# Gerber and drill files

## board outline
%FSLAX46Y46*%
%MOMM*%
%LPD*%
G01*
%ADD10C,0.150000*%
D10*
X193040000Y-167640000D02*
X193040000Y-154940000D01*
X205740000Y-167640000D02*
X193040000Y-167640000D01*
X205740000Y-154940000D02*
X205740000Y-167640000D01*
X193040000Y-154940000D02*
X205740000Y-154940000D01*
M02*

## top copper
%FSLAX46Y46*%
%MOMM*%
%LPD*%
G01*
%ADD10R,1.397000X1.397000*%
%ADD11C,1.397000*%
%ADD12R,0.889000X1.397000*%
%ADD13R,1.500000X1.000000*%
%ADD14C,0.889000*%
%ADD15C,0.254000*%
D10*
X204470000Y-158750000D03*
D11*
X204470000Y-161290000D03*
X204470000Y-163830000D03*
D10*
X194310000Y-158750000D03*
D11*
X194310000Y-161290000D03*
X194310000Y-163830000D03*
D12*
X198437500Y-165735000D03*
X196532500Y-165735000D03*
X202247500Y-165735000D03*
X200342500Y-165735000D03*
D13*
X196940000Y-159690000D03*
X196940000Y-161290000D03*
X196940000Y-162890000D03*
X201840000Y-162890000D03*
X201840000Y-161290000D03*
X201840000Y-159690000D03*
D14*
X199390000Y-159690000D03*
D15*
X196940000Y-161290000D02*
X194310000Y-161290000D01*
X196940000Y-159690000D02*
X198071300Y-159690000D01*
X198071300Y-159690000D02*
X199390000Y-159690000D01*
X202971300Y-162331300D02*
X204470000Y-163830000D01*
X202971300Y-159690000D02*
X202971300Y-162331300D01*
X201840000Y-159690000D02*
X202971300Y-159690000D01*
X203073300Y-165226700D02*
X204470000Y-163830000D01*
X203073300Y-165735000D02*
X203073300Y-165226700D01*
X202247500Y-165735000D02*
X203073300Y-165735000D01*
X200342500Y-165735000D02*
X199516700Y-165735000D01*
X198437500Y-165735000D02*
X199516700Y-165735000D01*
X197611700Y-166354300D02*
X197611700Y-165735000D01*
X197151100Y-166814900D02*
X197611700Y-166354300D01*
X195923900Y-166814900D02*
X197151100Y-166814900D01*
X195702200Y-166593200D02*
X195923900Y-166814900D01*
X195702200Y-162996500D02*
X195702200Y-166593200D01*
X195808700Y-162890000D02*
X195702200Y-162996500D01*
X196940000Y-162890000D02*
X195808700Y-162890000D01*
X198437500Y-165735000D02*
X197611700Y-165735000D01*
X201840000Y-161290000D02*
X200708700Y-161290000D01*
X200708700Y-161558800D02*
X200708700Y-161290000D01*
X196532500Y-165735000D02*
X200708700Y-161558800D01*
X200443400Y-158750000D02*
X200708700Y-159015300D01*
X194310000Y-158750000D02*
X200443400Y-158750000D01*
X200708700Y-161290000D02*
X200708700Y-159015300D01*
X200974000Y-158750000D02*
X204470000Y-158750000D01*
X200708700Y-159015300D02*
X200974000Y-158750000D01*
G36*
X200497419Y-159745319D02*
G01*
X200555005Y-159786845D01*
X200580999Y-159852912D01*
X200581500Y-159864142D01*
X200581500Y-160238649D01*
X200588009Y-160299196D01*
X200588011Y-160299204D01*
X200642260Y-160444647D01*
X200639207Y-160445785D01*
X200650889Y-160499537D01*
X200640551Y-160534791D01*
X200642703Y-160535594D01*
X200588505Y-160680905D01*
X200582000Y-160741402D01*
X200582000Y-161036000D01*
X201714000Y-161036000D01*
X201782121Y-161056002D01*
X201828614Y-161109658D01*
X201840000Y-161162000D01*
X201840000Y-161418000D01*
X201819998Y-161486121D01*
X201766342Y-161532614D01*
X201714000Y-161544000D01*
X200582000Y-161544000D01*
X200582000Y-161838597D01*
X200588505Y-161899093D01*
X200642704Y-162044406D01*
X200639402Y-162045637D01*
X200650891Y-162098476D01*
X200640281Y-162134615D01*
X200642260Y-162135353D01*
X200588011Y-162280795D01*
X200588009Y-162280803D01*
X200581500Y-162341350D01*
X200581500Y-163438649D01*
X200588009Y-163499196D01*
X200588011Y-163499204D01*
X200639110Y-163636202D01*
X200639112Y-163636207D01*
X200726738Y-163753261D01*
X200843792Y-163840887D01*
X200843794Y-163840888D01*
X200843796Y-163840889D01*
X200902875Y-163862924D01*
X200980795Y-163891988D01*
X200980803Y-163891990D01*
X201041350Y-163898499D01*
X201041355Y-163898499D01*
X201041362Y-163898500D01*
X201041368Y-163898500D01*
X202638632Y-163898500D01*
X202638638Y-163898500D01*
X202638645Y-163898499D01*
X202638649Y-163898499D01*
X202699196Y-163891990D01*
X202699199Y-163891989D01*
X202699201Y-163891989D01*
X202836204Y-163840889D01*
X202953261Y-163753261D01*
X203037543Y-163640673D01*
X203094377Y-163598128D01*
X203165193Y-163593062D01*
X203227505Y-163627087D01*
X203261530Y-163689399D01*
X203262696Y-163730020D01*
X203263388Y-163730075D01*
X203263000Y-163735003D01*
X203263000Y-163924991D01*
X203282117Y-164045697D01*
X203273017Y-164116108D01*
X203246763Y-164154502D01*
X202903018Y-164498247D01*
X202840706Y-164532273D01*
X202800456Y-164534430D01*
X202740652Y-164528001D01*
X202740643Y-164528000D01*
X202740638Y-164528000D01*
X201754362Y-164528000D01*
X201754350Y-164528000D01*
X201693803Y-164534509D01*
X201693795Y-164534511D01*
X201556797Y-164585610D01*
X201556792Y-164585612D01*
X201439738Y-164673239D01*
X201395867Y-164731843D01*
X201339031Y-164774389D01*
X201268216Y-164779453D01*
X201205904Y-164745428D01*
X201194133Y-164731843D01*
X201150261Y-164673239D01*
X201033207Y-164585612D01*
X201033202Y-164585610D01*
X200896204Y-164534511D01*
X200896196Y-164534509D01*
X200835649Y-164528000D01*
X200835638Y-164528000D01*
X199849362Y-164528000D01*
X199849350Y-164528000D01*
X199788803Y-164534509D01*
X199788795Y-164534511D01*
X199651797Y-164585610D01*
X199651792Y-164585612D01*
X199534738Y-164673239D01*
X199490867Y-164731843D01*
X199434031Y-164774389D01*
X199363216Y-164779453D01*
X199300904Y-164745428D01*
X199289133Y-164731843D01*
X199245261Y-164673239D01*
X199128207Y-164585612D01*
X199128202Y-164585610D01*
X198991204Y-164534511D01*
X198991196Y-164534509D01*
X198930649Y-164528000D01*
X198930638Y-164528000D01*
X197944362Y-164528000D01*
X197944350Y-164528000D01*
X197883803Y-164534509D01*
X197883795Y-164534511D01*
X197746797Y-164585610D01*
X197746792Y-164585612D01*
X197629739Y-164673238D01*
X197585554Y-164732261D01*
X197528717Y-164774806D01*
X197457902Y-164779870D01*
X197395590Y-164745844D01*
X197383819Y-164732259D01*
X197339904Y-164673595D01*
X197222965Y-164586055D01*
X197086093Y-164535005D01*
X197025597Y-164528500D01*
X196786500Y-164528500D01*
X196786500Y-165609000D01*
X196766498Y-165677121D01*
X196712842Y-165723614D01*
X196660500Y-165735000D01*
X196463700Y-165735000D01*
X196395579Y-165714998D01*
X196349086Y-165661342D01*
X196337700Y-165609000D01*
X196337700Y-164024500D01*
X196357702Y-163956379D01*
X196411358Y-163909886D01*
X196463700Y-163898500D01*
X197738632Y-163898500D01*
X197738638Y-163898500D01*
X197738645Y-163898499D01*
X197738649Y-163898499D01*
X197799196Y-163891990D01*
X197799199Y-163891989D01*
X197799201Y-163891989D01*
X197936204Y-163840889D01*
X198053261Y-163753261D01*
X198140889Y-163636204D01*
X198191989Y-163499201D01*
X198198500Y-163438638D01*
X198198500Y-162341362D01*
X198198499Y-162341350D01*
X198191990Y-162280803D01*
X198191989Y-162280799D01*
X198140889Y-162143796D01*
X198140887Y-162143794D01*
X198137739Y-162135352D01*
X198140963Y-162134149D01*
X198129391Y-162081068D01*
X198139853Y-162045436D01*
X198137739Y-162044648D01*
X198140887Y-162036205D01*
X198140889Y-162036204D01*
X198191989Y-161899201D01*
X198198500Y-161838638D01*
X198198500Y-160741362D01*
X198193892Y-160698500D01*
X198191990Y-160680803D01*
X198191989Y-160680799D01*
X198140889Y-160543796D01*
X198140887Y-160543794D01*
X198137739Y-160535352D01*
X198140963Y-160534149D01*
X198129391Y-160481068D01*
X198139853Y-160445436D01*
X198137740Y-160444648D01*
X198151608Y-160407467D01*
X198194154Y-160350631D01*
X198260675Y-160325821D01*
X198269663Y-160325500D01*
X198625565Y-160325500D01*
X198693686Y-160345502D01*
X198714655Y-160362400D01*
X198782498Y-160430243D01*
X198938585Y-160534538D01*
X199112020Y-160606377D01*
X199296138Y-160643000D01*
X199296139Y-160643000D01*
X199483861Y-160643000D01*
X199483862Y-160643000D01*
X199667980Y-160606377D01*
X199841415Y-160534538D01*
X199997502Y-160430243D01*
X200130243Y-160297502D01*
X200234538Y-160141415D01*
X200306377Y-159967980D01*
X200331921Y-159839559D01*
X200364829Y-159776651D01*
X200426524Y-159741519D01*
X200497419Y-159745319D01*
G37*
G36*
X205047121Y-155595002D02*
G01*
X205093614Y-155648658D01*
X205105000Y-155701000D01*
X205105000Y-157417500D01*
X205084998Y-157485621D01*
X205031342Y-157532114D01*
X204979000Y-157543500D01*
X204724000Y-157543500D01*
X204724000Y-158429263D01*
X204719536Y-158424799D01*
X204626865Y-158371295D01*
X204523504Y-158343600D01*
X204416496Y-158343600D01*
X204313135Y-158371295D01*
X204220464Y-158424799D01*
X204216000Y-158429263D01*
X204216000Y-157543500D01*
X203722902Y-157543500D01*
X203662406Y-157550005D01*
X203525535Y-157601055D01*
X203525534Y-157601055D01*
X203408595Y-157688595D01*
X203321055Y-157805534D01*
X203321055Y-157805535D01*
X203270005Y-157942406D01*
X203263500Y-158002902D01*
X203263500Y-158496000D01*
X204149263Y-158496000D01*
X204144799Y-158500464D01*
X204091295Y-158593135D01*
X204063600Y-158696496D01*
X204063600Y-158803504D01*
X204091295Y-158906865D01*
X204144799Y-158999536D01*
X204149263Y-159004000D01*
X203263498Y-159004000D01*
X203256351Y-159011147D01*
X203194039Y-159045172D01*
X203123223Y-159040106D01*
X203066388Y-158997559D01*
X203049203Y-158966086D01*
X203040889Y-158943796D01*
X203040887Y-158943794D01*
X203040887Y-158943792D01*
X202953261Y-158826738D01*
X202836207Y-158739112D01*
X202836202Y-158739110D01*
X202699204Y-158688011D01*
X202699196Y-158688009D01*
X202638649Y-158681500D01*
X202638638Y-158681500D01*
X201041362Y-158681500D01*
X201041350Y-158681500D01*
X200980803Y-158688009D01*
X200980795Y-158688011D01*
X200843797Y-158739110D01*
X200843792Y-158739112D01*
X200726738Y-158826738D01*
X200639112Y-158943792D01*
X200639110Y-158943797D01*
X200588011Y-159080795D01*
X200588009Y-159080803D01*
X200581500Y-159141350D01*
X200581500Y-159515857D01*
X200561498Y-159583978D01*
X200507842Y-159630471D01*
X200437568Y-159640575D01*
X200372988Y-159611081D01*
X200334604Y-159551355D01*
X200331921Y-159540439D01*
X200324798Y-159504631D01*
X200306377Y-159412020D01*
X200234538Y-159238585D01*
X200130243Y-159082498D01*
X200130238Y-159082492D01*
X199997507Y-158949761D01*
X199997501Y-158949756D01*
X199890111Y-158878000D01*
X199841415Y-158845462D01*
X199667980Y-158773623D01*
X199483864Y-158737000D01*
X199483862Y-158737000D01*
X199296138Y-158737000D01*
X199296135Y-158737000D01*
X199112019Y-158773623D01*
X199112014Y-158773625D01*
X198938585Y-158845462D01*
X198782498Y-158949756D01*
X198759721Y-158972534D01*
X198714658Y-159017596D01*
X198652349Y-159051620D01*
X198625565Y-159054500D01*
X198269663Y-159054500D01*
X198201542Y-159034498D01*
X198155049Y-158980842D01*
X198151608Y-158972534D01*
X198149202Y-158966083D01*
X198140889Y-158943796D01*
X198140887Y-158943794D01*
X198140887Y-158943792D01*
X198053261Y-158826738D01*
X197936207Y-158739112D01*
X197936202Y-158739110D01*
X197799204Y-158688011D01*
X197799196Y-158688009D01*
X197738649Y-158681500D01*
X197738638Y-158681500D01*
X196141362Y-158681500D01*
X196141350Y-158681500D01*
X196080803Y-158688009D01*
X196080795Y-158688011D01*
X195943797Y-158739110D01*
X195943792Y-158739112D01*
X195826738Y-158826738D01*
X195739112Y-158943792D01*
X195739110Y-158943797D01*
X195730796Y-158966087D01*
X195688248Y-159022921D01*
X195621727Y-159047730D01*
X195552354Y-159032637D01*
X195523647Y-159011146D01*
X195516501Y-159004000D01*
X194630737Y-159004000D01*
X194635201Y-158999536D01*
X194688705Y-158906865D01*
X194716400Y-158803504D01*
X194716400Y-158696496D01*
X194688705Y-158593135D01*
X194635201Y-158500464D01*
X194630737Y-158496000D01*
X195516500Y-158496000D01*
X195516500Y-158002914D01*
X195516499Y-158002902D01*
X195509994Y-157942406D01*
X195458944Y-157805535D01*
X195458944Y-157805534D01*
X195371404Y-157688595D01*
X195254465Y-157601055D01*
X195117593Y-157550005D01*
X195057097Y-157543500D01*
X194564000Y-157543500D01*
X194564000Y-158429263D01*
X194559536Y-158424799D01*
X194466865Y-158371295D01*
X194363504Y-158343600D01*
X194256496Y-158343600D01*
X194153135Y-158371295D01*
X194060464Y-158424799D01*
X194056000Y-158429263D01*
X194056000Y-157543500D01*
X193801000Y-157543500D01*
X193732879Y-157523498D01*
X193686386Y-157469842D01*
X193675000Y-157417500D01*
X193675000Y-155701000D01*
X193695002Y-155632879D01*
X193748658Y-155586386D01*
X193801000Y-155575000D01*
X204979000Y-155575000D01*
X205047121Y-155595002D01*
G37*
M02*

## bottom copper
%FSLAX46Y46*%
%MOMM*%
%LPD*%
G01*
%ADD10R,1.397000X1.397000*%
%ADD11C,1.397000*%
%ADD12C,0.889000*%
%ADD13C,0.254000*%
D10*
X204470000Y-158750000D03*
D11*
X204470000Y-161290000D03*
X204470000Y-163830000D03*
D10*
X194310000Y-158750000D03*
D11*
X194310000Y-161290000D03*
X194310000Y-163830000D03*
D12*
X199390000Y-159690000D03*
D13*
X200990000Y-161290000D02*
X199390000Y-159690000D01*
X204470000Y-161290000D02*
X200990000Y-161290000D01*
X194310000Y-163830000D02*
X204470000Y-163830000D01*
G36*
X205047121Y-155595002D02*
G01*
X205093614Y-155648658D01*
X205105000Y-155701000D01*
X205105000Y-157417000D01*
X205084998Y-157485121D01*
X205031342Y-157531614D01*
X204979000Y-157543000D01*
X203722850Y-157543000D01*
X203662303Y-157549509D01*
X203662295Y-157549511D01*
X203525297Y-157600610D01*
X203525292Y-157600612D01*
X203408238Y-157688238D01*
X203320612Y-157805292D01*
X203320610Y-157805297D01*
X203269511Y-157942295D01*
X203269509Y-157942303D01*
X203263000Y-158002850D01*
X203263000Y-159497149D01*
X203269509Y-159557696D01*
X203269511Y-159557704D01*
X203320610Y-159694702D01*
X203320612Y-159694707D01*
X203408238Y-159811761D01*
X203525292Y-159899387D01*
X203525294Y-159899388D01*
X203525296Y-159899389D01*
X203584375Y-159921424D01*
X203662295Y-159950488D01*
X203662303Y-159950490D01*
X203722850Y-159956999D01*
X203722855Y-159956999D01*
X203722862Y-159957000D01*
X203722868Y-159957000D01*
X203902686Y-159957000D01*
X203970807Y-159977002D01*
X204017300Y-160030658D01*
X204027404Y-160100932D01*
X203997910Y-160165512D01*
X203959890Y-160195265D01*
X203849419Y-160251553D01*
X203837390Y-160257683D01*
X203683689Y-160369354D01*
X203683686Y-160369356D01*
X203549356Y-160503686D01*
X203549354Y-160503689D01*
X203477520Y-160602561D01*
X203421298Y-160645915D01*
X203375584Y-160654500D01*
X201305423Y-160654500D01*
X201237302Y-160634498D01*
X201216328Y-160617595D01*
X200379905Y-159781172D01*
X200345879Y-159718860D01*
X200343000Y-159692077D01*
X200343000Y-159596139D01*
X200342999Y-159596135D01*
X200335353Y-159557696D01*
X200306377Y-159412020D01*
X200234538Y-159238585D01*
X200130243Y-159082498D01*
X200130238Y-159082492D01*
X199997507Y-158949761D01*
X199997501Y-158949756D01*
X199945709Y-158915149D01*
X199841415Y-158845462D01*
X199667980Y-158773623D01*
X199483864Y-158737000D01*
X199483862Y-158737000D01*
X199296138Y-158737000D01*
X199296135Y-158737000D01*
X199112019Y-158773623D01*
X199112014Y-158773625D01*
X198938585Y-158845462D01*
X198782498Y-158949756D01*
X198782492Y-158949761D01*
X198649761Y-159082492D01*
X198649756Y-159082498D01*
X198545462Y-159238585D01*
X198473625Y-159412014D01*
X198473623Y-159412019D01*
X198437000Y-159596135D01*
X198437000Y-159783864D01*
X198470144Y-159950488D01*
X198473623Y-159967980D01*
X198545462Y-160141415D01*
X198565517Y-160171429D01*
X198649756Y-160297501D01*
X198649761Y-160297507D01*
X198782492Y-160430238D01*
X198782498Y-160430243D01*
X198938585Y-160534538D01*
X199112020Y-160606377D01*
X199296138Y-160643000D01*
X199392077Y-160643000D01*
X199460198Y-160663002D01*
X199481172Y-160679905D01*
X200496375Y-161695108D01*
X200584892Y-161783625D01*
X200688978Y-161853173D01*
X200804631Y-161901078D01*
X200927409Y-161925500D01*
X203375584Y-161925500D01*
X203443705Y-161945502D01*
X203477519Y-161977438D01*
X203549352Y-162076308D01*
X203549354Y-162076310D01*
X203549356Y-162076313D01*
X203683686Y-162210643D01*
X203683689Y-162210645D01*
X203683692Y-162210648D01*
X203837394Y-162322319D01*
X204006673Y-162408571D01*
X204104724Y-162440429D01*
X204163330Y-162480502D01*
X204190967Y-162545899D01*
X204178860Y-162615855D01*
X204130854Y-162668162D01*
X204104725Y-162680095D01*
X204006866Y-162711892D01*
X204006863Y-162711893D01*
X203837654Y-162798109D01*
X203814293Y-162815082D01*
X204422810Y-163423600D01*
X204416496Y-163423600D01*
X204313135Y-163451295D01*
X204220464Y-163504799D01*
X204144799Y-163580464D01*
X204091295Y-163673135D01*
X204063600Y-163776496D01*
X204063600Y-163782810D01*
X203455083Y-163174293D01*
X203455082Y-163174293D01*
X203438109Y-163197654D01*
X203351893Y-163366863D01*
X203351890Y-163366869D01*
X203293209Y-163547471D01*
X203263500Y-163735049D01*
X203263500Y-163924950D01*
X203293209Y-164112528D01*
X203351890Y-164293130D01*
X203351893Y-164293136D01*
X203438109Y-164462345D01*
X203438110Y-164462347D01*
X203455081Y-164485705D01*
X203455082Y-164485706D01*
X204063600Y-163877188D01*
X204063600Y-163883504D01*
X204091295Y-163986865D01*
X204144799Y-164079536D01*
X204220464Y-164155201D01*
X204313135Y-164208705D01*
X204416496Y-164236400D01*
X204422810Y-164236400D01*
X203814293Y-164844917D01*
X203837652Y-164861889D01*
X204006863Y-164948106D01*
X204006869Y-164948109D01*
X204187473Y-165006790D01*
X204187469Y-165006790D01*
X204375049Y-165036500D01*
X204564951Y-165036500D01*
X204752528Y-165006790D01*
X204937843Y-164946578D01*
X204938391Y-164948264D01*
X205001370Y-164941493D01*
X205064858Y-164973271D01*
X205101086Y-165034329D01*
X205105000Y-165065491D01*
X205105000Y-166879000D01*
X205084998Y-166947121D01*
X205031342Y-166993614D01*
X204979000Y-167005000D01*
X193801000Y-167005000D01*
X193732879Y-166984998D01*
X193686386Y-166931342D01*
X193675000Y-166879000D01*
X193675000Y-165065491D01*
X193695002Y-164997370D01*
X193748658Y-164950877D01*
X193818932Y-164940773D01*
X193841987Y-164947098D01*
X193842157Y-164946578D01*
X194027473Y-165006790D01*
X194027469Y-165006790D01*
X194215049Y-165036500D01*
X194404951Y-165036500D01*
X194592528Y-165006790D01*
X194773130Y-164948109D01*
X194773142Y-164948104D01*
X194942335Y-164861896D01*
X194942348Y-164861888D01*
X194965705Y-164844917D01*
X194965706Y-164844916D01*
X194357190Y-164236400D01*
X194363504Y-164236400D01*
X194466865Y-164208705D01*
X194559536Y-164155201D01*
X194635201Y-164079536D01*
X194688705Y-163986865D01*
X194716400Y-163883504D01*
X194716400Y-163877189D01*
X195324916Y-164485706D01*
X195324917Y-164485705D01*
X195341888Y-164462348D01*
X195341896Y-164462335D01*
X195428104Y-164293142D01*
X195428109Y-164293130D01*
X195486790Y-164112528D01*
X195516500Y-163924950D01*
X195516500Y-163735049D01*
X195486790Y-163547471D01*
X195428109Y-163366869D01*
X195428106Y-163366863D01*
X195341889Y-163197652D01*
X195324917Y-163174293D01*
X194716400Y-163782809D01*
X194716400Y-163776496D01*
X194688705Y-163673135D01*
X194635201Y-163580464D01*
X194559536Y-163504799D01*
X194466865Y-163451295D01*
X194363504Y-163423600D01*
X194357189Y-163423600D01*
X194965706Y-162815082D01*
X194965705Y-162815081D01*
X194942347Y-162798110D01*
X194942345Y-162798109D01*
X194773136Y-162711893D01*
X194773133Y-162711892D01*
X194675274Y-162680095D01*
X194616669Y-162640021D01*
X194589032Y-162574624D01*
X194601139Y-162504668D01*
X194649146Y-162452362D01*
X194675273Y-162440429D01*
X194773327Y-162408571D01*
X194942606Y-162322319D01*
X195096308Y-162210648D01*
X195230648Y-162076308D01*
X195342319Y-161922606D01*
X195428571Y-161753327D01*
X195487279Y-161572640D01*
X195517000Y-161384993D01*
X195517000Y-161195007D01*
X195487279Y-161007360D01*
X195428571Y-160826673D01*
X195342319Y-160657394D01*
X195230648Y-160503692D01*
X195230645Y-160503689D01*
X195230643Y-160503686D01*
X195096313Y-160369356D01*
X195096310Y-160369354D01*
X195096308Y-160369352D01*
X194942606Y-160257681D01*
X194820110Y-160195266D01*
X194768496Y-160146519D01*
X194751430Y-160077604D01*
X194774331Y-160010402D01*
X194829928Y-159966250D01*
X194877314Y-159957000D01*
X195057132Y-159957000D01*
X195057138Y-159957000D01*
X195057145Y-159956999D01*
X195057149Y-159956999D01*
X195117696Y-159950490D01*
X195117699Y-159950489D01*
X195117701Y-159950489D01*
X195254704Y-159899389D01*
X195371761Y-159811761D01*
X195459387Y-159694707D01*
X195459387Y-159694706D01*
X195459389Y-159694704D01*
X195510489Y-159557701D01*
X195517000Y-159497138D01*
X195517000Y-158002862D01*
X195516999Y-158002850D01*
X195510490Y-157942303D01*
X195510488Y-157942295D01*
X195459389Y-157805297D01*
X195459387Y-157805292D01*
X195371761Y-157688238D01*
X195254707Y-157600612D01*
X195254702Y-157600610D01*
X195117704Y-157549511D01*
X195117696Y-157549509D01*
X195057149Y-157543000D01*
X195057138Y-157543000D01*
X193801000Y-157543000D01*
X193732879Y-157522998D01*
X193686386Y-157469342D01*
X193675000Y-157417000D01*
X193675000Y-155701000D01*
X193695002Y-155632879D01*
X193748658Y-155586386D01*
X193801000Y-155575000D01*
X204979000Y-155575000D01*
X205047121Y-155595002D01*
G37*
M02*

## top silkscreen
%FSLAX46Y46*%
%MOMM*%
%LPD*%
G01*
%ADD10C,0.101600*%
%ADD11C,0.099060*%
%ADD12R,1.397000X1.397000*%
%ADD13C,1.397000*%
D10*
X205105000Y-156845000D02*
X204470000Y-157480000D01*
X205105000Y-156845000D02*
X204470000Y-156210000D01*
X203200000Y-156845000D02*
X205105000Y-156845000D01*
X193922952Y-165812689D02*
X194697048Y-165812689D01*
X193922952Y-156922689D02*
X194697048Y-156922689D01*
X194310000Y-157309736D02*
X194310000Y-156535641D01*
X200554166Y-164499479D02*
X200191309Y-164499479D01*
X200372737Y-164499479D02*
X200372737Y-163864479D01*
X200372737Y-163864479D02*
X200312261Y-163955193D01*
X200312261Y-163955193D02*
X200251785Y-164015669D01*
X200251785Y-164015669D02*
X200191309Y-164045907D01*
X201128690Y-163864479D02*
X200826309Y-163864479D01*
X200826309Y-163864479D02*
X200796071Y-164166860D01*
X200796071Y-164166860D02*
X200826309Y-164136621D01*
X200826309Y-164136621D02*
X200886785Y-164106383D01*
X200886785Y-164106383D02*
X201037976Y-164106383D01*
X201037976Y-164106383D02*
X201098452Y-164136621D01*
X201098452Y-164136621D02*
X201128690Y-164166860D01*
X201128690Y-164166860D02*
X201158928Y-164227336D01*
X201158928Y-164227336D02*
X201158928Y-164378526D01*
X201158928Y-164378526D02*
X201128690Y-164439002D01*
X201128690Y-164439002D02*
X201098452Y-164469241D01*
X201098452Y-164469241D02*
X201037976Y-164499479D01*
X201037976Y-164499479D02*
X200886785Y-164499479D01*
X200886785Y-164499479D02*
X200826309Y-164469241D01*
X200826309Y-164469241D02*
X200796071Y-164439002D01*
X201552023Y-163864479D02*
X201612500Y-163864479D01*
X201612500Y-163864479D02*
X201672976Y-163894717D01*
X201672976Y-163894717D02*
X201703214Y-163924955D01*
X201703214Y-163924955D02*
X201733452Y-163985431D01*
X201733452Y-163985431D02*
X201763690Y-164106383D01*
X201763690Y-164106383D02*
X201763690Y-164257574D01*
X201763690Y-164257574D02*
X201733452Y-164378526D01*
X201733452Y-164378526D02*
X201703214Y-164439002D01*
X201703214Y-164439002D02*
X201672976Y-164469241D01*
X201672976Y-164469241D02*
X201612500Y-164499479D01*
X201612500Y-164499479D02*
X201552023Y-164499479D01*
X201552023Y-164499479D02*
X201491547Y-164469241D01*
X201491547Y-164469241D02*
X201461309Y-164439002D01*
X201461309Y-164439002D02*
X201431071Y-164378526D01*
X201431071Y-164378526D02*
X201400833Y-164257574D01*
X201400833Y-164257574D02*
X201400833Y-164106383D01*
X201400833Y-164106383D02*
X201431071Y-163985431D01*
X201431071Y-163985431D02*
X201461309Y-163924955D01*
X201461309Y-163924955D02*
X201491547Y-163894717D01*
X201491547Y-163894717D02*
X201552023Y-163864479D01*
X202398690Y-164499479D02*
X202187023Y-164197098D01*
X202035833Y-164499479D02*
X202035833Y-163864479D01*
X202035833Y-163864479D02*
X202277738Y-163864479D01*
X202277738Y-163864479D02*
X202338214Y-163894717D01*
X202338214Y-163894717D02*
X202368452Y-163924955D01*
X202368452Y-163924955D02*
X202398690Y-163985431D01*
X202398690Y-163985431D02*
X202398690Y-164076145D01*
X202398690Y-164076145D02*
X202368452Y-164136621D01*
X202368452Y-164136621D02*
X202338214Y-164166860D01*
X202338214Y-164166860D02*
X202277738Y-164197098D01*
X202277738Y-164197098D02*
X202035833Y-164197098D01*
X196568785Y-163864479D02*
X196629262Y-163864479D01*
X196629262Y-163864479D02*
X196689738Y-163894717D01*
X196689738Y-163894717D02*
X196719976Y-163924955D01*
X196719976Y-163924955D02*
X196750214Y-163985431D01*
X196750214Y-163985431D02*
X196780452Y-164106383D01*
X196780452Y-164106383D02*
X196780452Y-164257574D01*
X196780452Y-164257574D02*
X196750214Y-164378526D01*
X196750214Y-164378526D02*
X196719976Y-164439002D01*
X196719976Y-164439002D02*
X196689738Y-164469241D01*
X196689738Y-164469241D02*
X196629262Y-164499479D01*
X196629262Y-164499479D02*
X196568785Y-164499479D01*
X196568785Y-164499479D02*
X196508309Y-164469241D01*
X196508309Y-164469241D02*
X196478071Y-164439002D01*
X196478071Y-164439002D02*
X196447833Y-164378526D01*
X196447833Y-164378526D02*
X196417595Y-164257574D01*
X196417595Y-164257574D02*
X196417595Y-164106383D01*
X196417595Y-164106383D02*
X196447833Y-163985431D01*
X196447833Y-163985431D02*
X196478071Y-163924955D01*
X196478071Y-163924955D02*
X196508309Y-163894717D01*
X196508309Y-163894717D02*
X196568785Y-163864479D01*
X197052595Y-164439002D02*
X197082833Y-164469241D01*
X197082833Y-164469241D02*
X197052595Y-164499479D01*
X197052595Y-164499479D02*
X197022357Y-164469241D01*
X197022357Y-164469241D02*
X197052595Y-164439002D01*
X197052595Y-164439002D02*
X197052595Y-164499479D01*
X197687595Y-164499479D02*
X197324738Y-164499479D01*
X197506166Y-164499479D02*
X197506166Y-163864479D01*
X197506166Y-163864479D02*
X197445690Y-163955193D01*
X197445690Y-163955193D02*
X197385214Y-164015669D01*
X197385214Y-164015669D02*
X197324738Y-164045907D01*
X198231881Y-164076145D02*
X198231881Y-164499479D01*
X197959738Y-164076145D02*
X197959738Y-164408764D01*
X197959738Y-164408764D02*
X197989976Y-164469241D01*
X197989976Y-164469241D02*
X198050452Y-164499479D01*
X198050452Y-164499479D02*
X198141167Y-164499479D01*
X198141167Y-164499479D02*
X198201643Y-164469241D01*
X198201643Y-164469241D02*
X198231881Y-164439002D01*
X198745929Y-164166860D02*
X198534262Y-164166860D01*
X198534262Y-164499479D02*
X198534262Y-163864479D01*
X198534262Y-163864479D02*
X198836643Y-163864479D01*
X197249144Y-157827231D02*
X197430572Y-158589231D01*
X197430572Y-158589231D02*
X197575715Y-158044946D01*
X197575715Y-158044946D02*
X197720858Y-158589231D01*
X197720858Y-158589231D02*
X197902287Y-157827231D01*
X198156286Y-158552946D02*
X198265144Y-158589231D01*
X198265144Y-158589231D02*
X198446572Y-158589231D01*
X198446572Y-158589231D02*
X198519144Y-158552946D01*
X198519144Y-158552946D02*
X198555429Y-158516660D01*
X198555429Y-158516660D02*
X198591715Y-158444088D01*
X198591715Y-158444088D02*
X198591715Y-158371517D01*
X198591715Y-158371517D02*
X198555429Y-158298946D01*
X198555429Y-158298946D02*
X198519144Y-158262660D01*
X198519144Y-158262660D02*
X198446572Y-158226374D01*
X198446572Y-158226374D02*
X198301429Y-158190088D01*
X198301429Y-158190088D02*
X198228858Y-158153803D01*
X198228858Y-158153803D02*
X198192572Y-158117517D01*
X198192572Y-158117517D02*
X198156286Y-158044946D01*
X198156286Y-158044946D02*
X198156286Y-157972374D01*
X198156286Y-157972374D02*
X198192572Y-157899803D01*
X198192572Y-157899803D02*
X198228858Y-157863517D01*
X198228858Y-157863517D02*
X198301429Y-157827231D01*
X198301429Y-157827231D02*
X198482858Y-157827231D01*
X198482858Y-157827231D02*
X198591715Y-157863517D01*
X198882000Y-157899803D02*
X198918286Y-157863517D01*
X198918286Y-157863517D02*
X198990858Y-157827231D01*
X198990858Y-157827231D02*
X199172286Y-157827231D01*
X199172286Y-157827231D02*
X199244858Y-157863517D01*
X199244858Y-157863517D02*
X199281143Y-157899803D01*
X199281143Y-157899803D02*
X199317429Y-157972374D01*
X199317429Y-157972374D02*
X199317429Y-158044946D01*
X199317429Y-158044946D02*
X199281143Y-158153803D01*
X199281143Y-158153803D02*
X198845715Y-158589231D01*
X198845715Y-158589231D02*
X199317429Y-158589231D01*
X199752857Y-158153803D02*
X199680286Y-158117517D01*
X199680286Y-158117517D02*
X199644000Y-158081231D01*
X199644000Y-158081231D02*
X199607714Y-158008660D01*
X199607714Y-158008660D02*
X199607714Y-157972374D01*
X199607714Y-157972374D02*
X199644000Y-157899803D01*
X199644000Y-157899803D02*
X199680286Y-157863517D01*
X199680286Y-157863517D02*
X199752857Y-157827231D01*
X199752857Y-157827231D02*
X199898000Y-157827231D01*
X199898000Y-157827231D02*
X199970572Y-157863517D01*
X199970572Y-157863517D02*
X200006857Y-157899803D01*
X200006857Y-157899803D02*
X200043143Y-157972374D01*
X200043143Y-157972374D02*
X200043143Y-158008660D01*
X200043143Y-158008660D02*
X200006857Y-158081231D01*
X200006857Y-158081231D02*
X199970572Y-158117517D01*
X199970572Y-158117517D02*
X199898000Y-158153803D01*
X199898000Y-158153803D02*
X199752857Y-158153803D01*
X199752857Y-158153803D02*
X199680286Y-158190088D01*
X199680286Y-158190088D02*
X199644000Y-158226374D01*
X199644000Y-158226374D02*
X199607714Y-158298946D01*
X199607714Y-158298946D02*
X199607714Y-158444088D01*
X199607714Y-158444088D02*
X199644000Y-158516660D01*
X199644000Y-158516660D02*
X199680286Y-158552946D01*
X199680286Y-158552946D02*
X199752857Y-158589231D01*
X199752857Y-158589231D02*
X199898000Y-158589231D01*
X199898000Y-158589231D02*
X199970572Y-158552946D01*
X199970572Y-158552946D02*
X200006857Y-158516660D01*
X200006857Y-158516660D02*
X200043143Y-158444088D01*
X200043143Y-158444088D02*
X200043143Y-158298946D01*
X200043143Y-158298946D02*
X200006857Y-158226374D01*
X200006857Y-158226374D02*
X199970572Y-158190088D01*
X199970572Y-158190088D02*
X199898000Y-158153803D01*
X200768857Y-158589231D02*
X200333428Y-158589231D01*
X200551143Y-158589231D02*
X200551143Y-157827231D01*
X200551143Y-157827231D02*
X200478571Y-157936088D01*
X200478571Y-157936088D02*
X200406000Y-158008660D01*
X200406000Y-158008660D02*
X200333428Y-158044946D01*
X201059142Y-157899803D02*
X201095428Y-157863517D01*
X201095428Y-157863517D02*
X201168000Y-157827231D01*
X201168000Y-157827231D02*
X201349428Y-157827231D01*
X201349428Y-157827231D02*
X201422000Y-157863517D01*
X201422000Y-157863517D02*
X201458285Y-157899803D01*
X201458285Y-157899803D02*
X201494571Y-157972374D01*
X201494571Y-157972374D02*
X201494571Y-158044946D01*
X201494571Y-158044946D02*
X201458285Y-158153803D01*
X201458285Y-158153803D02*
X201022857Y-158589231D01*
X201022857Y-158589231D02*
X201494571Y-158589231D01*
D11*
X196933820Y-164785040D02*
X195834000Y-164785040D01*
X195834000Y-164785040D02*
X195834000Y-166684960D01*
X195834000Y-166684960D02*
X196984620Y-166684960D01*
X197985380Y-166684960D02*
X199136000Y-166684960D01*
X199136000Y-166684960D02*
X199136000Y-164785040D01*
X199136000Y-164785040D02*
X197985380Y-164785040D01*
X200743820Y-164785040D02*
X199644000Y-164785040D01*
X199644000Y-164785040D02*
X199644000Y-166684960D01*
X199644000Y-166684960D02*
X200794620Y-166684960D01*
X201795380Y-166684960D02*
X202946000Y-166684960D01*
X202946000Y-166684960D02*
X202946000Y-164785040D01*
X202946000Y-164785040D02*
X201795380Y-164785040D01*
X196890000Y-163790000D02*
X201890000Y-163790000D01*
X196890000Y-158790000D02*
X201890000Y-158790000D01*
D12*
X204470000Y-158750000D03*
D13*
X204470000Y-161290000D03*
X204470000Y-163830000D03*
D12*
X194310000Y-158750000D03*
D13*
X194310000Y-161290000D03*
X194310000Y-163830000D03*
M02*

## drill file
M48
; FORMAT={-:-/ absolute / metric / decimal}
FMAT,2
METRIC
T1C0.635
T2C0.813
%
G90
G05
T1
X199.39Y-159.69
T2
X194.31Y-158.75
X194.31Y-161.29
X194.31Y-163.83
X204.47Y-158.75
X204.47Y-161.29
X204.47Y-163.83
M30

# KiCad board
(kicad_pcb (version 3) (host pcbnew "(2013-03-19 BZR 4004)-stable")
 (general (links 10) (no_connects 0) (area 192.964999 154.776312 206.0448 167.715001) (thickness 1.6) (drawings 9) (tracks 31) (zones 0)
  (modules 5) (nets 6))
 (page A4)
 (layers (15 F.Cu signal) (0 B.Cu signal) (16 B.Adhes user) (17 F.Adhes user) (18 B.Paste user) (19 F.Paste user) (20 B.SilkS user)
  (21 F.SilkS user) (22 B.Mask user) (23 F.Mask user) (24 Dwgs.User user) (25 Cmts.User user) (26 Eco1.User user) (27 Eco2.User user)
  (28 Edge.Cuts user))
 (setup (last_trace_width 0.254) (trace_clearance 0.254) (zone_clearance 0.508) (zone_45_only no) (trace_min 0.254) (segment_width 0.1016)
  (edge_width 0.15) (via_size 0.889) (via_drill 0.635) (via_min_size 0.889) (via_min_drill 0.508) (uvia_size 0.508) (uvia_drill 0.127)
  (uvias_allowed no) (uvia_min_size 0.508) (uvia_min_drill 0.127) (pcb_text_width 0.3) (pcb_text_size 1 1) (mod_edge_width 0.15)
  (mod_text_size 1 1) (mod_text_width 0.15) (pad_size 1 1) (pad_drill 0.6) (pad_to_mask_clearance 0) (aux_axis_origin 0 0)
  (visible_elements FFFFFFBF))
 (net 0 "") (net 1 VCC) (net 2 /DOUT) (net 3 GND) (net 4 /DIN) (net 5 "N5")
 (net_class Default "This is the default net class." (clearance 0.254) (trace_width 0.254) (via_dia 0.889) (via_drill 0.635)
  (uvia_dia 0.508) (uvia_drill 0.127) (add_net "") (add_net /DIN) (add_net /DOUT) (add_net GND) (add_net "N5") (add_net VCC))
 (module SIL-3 (layer F.Cu) (at 204.47 161.29 270)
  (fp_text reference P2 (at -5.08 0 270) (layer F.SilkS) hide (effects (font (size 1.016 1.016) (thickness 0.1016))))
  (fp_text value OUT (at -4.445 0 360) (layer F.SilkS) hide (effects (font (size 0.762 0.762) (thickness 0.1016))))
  (pad 1 thru_hole rect (at -2.54 0 270) (size 1.397 1.397) (drill 0.8128) (layers *.Cu *.Mask F.SilkS) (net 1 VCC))
  (pad 2 thru_hole circle (at 0 0 270) (size 1.397 1.397) (drill 0.8128) (layers *.Cu *.Mask F.SilkS) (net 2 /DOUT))
  (pad 3 thru_hole circle (at 2.54 0 270) (size 1.397 1.397) (drill 0.8128) (layers *.Cu *.Mask F.SilkS) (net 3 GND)))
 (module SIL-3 (layer F.Cu) (at 194.31 161.29 270)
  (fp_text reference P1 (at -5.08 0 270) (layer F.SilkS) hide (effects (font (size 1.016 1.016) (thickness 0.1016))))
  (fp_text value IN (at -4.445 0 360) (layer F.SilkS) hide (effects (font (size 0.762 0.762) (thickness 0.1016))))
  (pad 1 thru_hole rect (at -2.54 0 270) (size 1.397 1.397) (drill 0.8128) (layers *.Cu *.Mask F.SilkS) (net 1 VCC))
  (pad 2 thru_hole circle (at 0 0 270) (size 1.397 1.397) (drill 0.8128) (layers *.Cu *.Mask F.SilkS) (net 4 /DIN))
  (pad 3 thru_hole circle (at 2.54 0 270) (size 1.397 1.397) (drill 0.8128) (layers *.Cu *.Mask F.SilkS) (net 3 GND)))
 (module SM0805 (layer F.Cu) (at 197.485 165.735 180)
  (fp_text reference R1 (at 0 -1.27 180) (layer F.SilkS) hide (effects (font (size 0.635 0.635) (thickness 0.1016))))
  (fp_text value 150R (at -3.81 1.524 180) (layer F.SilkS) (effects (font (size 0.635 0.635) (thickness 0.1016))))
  (fp_line (start 0.55118 0.94996) (end 1.651 0.94996) (layer F.SilkS) (width 0.09906))
  (fp_line (start 1.651 0.94996) (end 1.651 -0.94996) (layer F.SilkS) (width 0.09906))
  (fp_line (start 1.651 -0.94996) (end 0.50038 -0.94996) (layer F.SilkS) (width 0.09906))
  (fp_line (start -0.50038 -0.94996) (end -1.651 -0.94996) (layer F.SilkS) (width 0.09906))
  (fp_line (start -1.651 -0.94996) (end -1.651 0.94996) (layer F.SilkS) (width 0.09906))
  (fp_line (start -1.651 0.94996) (end -0.50038 0.94996) (layer F.SilkS) (width 0.09906))
  (pad 1 smd rect (at -0.9525 0 180) (size 0.889 1.397) (layers F.Cu F.Paste F.Mask) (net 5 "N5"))
  (pad 2 smd rect (at 0.9525 0 180) (size 0.889 1.397) (layers F.Cu F.Paste F.Mask) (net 1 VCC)))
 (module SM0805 (layer F.Cu) (at 201.295 165.735 180)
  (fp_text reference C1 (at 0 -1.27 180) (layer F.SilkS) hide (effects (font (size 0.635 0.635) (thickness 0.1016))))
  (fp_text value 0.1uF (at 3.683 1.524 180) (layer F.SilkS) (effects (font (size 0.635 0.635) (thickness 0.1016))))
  (fp_line (start 0.55118 0.94996) (end 1.651 0.94996) (layer F.SilkS) (width 0.09906))
  (fp_line (start 1.651 0.94996) (end 1.651 -0.94996) (layer F.SilkS) (width 0.09906))
  (fp_line (start 1.651 -0.94996) (end 0.50038 -0.94996) (layer F.SilkS) (width 0.09906))
  (fp_line (start -0.50038 -0.94996) (end -1.651 -0.94996) (layer F.SilkS) (width 0.09906))
  (fp_line (start -1.651 -0.94996) (end -1.651 0.94996) (layer F.SilkS) (width 0.09906))
  (fp_line (start -1.651 0.94996) (end -0.50038 0.94996) (layer F.SilkS) (width 0.09906))
  (pad 1 smd rect (at -0.9525 0 180) (size 0.889 1.397) (layers F.Cu F.Paste F.Mask) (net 3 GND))
  (pad 2 smd rect (at 0.9525 0 180) (size 0.889 1.397) (layers F.Cu F.Paste F.Mask) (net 5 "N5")))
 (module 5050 (layer F.Cu) (at 199.39 161.29)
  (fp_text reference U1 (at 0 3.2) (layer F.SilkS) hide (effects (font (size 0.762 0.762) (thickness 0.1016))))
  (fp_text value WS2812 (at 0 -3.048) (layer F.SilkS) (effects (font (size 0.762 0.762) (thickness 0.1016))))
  (fp_line (start -2.5 2.5) (end 2.5 2.5) (layer F.SilkS) (width 0.09906))
  (fp_line (start -2.5 -2.5) (end 2.5 -2.5) (layer F.SilkS) (width 0.09906))
  (pad 1 smd rect (at -2.45 -1.6) (size 1.5 1) (layers F.Cu F.Paste F.Mask) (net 2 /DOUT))
  (pad 2 smd rect (at -2.45 0) (size 1.5 1) (layers F.Cu F.Paste F.Mask) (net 4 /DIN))
  (pad 3 smd rect (at -2.45 1.6) (size 1.5 1) (layers F.Cu F.Paste F.Mask) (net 5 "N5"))
  (pad 4 smd rect (at 2.45 1.6) (size 1.5 1) (layers F.Cu F.Paste F.Mask))
  (pad 5 smd rect (at 2.45 0) (size 1.5 1) (layers F.Cu F.Paste F.Mask) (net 1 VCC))
  (pad 6 smd rect (at 2.45 -1.6) (size 1.5 1) (layers F.Cu F.Paste F.Mask) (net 3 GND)))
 (gr_line (start 205.105 156.845) (end 204.47 157.48) (angle 90) (layer F.SilkS) (width 0.1016))
 (gr_line (start 205.105 156.845) (end 204.47 156.21) (angle 90) (layer F.SilkS) (width 0.1016))
 (gr_line (start 203.2 156.845) (end 205.105 156.845) (angle 90) (layer F.SilkS) (width 0.1016))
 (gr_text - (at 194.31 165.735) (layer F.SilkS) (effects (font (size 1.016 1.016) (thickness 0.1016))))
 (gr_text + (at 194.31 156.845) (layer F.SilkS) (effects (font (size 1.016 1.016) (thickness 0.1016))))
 (gr_line (start 193.04 167.64) (end 193.04 154.94) (angle 90) (layer Edge.Cuts) (width 0.15))
 (gr_line (start 205.74 167.64) (end 193.04 167.64) (angle 90) (layer Edge.Cuts) (width 0.15))
 (gr_line (start 205.74 154.94) (end 205.74 167.64) (angle 90) (layer Edge.Cuts) (width 0.15))
 (gr_line (start 193.04 154.94) (end 205.74 154.94) (angle 90) (layer Edge.Cuts) (width 0.15))
 (segment (start 196.94 161.29) (end 194.31 161.29) (width 0.254) (layer F.Cu) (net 4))
 (via (at 199.39 159.69) (size 0.889) (layers F.Cu B.Cu) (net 2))
 (segment (start 196.94 159.69) (end 198.0713 159.69) (width 0.254) (layer F.Cu) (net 2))
 (segment (start 200.99 161.29) (end 199.39 159.69) (width 0.254) (layer B.Cu) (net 2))
 (segment (start 204.47 161.29) (end 200.99 161.29) (width 0.254) (layer B.Cu) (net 2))
 (segment (start 198.0713 159.69) (end 199.39 159.69) (width 0.254) (layer F.Cu) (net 2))
 (segment (start 202.9713 162.3313) (end 204.47 163.83) (width 0.254) (layer F.Cu) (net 3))
 (segment (start 202.9713 159.69) (end 202.9713 162.3313) (width 0.254) (layer F.Cu) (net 3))
 (segment (start 201.84 159.69) (end 202.9713 159.69) (width 0.254) (layer F.Cu) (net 3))
 (segment (start 203.0733 165.2267) (end 204.47 163.83) (width 0.254) (layer F.Cu) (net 3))
 (segment (start 203.0733 165.735) (end 203.0733 165.2267) (width 0.254) (layer F.Cu) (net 3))
 (segment (start 202.2475 165.735) (end 203.0733 165.735) (width 0.254) (layer F.Cu) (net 3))
 (segment (start 194.31 163.83) (end 204.47 163.83) (width 0.254) (layer B.Cu) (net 3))
 (segment (start 200.3425 165.735) (end 199.5167 165.735) (width 0.254) (layer F.Cu) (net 5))
 (segment (start 198.4375 165.735) (end 199.5167 165.735) (width 0.254) (layer F.Cu) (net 5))
 (segment (start 197.6117 166.3543) (end 197.6117 165.735) (width 0.254) (layer F.Cu) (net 5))
 (segment (start 197.1511 166.8149) (end 197.6117 166.3543) (width 0.254) (layer F.Cu) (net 5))
 (segment (start 195.9239 166.8149) (end 197.1511 166.8149) (width 0.254) (layer F.Cu) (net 5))
 (segment (start 195.7022 166.5932) (end 195.9239 166.8149) (width 0.254) (layer F.Cu) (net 5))
 (segment (start 195.7022 162.9965) (end 195.7022 166.5932) (width 0.254) (layer F.Cu) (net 5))
 (segment (start 195.8087 162.89) (end 195.7022 162.9965) (width 0.254) (layer F.Cu) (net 5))
 (segment (start 196.94 162.89) (end 195.8087 162.89) (width 0.254) (layer F.Cu) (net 5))
 (segment (start 198.4375 165.735) (end 197.6117 165.735) (width 0.254) (layer F.Cu) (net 5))
 (segment (start 201.84 161.29) (end 200.7087 161.29) (width 0.254) (layer F.Cu) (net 1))
 (segment (start 200.7087 161.5588) (end 200.7087 161.29) (width 0.254) (layer F.Cu) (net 1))
 (segment (start 196.5325 165.735) (end 200.7087 161.5588) (width 0.254) (layer F.Cu) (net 1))
 (segment (start 200.4434 158.75) (end 200.7087 159.0153) (width 0.254) (layer F.Cu) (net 1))
 (segment (start 194.31 158.75) (end 200.4434 158.75) (width 0.254) (layer F.Cu) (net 1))
 (segment (start 200.7087 161.29) (end 200.7087 159.0153) (width 0.254) (layer F.Cu) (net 1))
 (segment (start 200.974 158.75) (end 204.47 158.75) (width 0.254) (layer F.Cu) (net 1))
 (segment (start 200.7087 159.0153) (end 200.974 158.75) (width 0.254) (layer F.Cu) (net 1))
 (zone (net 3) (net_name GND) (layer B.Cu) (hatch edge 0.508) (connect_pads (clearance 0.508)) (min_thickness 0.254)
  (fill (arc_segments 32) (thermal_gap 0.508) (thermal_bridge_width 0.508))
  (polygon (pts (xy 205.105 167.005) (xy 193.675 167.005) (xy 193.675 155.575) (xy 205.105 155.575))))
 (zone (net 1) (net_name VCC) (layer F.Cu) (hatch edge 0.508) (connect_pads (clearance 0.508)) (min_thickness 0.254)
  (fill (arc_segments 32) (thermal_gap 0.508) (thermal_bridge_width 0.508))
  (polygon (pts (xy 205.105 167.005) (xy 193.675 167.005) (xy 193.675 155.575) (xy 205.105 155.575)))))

